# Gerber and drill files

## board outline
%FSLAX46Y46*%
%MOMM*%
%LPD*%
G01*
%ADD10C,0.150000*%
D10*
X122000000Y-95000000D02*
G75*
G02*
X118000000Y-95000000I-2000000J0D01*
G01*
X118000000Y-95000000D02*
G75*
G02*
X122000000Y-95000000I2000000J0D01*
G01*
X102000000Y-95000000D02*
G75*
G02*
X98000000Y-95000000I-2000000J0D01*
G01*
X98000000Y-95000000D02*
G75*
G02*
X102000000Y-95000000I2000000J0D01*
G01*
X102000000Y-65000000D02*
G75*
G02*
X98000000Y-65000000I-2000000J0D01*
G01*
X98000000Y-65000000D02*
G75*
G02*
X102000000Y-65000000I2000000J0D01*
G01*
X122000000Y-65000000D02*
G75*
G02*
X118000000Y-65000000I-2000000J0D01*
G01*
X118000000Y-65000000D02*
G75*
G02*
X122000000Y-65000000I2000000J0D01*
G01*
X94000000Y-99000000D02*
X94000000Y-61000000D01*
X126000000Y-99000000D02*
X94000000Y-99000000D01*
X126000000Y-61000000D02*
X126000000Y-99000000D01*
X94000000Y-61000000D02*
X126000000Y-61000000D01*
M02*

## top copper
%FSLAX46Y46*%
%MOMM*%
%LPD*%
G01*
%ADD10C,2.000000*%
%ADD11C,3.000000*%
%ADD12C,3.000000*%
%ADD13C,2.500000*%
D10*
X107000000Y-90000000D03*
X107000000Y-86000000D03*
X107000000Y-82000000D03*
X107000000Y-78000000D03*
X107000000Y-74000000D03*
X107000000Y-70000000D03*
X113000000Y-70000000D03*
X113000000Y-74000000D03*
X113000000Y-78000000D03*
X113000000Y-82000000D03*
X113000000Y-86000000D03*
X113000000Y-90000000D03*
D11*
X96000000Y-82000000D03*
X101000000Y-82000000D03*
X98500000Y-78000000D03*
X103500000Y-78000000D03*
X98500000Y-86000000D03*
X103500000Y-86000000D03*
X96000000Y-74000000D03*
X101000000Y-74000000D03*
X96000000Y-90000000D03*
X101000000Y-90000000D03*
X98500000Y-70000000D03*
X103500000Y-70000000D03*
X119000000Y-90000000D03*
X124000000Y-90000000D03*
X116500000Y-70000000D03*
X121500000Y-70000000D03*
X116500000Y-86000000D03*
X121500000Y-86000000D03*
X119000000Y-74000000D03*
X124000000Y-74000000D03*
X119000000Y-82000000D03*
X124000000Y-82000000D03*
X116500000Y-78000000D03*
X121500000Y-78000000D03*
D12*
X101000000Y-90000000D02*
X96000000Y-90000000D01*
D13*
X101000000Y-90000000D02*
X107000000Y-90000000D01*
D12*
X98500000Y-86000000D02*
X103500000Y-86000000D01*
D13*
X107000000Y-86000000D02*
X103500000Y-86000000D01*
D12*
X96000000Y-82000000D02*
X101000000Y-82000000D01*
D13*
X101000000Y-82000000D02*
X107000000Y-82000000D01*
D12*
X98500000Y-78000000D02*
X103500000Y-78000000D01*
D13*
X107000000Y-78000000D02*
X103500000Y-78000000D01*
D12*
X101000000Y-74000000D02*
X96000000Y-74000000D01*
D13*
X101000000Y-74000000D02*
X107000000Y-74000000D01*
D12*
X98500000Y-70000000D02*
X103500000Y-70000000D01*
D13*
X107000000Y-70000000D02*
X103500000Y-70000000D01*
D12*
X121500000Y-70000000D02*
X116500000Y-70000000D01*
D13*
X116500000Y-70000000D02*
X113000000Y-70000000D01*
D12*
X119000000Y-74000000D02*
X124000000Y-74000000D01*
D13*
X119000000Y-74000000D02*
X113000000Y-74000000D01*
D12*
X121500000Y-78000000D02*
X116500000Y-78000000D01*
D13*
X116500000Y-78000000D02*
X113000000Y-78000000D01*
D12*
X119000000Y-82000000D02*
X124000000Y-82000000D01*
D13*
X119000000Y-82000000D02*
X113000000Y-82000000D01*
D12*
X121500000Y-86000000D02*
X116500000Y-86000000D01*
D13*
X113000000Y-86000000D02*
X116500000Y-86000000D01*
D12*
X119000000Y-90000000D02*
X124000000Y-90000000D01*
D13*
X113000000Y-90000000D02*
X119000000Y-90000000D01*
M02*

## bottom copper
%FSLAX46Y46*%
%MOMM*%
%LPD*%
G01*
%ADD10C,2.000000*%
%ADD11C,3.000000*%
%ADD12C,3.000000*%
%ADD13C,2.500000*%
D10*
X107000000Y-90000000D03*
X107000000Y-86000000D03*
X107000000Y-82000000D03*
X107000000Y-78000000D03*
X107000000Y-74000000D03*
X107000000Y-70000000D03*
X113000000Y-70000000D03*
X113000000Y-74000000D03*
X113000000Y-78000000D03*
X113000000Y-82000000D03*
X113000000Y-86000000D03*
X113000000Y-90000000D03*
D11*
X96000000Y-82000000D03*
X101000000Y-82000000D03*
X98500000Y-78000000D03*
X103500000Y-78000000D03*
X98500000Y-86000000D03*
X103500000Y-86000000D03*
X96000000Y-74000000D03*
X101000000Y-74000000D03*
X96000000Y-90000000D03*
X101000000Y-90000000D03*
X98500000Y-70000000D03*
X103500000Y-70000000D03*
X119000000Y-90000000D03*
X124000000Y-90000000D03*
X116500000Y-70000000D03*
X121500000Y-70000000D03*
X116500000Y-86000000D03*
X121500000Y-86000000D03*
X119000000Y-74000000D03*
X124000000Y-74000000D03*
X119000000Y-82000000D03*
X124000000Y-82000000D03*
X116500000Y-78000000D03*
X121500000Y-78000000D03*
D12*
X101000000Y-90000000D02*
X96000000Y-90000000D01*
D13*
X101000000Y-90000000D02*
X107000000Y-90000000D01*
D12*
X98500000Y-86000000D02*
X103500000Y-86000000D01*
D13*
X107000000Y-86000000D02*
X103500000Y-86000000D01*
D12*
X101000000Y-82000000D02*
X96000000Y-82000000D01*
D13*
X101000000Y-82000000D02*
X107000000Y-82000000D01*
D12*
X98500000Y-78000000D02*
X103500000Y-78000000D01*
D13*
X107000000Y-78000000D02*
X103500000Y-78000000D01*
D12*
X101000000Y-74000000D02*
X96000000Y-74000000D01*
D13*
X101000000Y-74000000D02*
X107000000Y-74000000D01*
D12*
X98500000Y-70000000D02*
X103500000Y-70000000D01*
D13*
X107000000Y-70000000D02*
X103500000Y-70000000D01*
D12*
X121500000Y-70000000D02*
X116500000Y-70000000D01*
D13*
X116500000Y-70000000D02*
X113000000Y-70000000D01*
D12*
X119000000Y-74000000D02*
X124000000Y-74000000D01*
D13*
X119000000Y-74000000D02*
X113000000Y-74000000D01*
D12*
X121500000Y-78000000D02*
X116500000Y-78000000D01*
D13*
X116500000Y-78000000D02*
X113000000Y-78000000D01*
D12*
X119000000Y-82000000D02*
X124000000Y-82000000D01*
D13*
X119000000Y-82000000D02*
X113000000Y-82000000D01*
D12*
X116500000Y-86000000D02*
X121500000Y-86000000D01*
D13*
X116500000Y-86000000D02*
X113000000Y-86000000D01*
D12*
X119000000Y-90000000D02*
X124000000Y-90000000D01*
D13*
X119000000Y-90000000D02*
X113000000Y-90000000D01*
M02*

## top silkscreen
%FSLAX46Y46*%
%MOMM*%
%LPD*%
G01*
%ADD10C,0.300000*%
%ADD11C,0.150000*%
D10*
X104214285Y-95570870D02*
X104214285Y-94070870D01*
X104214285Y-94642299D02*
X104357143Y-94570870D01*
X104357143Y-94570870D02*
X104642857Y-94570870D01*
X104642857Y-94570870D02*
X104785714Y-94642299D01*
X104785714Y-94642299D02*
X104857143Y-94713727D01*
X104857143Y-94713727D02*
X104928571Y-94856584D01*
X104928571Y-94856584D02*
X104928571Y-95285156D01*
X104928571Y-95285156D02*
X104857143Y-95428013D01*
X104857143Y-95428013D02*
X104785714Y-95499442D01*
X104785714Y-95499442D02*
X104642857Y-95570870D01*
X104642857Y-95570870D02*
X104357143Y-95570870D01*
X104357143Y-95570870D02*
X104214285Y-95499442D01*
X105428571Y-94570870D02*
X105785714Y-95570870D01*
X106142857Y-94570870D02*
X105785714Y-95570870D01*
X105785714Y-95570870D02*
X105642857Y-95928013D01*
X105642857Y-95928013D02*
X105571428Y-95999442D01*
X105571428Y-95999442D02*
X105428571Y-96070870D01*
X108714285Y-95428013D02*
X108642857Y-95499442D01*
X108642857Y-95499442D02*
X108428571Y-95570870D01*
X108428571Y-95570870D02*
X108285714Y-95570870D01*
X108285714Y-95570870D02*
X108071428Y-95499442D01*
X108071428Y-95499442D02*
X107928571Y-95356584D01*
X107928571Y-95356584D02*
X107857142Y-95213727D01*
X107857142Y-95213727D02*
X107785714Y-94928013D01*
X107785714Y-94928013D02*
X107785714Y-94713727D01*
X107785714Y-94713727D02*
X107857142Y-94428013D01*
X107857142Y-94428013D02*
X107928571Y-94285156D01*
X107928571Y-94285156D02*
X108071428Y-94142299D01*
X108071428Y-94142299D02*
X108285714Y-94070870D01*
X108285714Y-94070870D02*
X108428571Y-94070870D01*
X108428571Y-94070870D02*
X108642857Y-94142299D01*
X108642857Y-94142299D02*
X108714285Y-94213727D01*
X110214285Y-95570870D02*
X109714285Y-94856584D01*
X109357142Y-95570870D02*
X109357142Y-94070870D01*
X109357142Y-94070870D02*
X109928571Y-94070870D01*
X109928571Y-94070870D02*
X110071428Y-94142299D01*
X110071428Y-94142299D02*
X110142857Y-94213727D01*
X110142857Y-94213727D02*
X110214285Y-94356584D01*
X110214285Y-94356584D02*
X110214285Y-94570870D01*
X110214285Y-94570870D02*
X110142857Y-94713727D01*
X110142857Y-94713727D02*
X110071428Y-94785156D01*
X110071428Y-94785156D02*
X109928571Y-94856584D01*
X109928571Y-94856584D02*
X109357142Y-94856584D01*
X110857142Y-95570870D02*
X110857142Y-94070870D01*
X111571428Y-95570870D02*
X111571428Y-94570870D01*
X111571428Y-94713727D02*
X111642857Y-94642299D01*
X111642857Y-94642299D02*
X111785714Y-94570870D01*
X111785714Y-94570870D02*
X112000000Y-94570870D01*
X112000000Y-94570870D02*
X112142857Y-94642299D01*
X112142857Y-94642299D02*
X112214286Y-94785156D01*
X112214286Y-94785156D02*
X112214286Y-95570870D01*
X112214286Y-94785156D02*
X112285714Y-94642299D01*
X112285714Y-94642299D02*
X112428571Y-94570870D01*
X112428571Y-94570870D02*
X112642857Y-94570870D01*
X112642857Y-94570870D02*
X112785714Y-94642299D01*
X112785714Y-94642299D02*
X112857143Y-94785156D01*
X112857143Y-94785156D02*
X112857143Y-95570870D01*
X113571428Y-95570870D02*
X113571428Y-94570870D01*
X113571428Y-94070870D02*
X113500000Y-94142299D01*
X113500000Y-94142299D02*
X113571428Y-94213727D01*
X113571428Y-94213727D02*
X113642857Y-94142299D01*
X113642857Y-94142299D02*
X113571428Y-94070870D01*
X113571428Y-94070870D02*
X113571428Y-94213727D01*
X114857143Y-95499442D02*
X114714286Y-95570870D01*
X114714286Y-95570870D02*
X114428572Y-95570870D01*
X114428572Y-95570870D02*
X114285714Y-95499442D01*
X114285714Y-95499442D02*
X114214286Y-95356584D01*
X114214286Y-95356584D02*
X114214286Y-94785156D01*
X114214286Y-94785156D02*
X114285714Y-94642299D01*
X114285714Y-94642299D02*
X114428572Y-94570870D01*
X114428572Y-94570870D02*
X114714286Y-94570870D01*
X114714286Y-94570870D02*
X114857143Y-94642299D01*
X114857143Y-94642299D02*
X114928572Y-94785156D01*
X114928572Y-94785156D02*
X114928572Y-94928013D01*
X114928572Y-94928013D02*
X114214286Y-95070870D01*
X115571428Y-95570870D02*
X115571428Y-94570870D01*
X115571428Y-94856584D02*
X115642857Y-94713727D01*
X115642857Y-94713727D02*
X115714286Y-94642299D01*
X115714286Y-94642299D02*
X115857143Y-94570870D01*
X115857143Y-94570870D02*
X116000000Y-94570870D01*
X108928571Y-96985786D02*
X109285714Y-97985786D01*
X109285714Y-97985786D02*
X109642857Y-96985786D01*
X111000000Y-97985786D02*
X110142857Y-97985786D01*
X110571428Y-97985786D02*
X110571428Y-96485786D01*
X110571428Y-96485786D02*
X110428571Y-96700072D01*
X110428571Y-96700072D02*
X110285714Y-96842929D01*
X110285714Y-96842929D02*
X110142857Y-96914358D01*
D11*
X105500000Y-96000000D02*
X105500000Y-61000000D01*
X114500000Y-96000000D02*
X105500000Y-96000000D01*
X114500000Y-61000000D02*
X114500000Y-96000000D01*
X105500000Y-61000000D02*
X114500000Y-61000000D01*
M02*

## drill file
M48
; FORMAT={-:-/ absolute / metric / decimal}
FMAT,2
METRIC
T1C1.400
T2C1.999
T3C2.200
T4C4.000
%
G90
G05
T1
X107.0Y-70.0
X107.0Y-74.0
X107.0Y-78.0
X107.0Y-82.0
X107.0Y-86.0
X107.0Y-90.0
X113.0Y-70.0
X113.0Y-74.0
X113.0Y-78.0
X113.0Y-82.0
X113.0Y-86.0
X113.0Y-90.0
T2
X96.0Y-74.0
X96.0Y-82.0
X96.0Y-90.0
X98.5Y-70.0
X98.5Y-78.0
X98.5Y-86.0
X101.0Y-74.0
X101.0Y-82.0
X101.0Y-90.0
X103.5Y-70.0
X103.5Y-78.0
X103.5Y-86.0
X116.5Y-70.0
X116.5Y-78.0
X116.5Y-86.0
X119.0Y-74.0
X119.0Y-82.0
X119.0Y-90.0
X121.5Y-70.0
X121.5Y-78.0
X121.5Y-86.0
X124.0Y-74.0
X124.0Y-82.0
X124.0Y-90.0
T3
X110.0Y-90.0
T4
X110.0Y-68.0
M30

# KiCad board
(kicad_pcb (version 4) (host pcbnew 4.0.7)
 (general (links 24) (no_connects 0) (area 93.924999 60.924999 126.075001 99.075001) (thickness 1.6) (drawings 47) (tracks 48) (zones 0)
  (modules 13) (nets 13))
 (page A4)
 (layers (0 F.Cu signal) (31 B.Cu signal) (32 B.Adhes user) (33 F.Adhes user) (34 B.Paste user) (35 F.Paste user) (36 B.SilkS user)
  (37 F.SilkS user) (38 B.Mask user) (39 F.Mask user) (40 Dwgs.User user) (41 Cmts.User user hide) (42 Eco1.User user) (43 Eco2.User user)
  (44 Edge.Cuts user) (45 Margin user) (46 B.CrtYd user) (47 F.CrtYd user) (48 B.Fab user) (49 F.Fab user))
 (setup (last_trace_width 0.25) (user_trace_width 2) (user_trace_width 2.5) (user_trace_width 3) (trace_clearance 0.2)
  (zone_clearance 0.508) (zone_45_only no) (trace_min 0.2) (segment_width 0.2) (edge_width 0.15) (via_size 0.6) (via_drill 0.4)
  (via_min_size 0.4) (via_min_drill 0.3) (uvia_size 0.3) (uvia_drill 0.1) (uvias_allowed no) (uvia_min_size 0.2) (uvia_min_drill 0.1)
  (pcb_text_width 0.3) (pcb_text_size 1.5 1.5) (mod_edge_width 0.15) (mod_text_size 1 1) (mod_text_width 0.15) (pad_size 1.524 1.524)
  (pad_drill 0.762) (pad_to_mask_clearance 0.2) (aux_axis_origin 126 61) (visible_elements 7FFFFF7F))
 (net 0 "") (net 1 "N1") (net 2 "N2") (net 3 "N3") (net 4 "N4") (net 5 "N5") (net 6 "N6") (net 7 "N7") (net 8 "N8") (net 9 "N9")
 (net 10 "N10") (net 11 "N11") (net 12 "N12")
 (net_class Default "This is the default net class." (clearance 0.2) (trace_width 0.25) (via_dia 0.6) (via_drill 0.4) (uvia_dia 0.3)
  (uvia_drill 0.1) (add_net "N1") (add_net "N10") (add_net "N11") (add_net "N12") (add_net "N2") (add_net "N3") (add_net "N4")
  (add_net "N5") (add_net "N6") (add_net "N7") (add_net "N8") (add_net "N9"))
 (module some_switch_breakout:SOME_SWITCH (layer F.Cu) (at 110 80)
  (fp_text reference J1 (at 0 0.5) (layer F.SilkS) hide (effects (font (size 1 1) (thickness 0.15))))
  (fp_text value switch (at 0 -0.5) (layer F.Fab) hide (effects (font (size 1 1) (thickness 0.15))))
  (fp_line (start -4.5 16) (end -4.5 -19) (layer F.SilkS) (width 0.15))
  (fp_line (start 4.5 16) (end -4.5 16) (layer F.SilkS) (width 0.15))
  (fp_line (start 4.5 -19) (end 4.5 16) (layer F.SilkS) (width 0.15))
  (fp_line (start -4.5 -19) (end 4.5 -19) (layer F.SilkS) (width 0.15))
  (pad 1 thru_hole circle (at -3 10) (size 2 2) (drill 1.4) (layers *.Cu *.Mask) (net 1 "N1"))
  (pad 2 thru_hole circle (at -3 6) (size 2 2) (drill 1.4) (layers *.Cu *.Mask) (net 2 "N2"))
  (pad 3 thru_hole circle (at -3 2) (size 2 2) (drill 1.4) (layers *.Cu *.Mask) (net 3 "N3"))
  (pad 4 thru_hole circle (at -3 -2) (size 2 2) (drill 1.4) (layers *.Cu *.Mask) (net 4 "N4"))
  (pad 5 thru_hole circle (at -3 -6) (size 2 2) (drill 1.4) (layers *.Cu *.Mask) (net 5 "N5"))
  (pad 6 thru_hole circle (at -3 -10) (size 2 2) (drill 1.4) (layers *.Cu *.Mask) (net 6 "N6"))
  (pad 7 thru_hole circle (at 3 -10) (size 2 2) (drill 1.4) (layers *.Cu *.Mask) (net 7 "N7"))
  (pad 8 thru_hole circle (at 3 -6) (size 2 2) (drill 1.4) (layers *.Cu *.Mask) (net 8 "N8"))
  (pad 9 thru_hole circle (at 3 -2) (size 2 2) (drill 1.4) (layers *.Cu *.Mask) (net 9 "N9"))
  (pad 10 thru_hole circle (at 3 2) (size 2 2) (drill 1.4) (layers *.Cu *.Mask) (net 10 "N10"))
  (pad 11 thru_hole circle (at 3 6) (size 2 2) (drill 1.4) (layers *.Cu *.Mask) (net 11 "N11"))
  (pad 12 thru_hole circle (at 3 10) (size 2 2) (drill 1.4) (layers *.Cu *.Mask) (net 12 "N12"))
  (pad "" np_thru_hole circle (at 0 10) (size 2.2 2.2) (drill 2.2) (layers *.Cu *.Mask))
  (pad "" np_thru_hole circle (at 0 -12) (size 4 4) (drill 4) (layers *.Cu *.Mask)))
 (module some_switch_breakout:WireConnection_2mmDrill (layer F.Cu) (at 98.5 82)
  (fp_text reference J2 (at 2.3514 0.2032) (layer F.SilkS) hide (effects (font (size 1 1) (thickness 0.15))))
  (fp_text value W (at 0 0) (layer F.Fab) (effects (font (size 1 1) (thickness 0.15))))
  (pad 1 thru_hole circle (at -2.5 0) (size 3 3) (drill 1.99898) (layers *.Cu *.Mask) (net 3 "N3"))
  (pad 2 thru_hole circle (at 2.5 0) (size 3 3) (drill 1.99898) (layers *.Cu *.Mask) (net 3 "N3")))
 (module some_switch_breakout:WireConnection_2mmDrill (layer F.Cu) (at 101 78)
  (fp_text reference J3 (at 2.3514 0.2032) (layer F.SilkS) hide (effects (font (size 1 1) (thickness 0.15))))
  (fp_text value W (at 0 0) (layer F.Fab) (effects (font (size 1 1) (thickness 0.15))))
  (pad 1 thru_hole circle (at -2.5 0) (size 3 3) (drill 1.99898) (layers *.Cu *.Mask) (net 4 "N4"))
  (pad 2 thru_hole circle (at 2.5 0) (size 3 3) (drill 1.99898) (layers *.Cu *.Mask) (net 4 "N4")))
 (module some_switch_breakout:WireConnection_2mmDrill (layer F.Cu) (at 101 86)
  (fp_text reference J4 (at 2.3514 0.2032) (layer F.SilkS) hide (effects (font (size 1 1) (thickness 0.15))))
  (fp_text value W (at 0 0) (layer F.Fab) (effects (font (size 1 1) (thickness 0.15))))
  (pad 1 thru_hole circle (at -2.5 0) (size 3 3) (drill 1.99898) (layers *.Cu *.Mask) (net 2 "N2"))
  (pad 2 thru_hole circle (at 2.5 0) (size 3 3) (drill 1.99898) (layers *.Cu *.Mask) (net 2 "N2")))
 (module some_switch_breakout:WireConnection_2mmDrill (layer F.Cu) (at 98.5 74)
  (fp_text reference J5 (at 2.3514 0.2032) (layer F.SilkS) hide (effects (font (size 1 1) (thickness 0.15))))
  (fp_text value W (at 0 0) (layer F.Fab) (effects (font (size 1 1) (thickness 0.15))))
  (pad 1 thru_hole circle (at -2.5 0) (size 3 3) (drill 1.99898) (layers *.Cu *.Mask) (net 5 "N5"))
  (pad 2 thru_hole circle (at 2.5 0) (size 3 3) (drill 1.99898) (layers *.Cu *.Mask) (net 5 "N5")))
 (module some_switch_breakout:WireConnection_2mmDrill (layer F.Cu) (at 98.5 90)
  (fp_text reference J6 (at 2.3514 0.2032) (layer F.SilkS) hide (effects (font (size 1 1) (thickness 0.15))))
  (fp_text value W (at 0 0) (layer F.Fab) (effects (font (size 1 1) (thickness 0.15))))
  (pad 1 thru_hole circle (at -2.5 0) (size 3 3) (drill 1.99898) (layers *.Cu *.Mask) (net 1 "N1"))
  (pad 2 thru_hole circle (at 2.5 0) (size 3 3) (drill 1.99898) (layers *.Cu *.Mask) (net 1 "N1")))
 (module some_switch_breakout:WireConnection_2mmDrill (layer F.Cu) (at 101 70)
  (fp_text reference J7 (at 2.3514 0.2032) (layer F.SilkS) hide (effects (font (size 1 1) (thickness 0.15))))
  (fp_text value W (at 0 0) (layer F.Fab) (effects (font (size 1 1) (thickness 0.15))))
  (pad 1 thru_hole circle (at -2.5 0) (size 3 3) (drill 1.99898) (layers *.Cu *.Mask) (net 6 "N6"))
  (pad 2 thru_hole circle (at 2.5 0) (size 3 3) (drill 1.99898) (layers *.Cu *.Mask) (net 6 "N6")))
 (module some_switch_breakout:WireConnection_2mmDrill (layer F.Cu) (at 121.5 90)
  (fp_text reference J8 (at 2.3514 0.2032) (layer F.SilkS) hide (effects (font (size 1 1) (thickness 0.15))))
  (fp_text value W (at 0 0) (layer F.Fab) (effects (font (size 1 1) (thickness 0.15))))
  (pad 1 thru_hole circle (at -2.5 0) (size 3 3) (drill 1.99898) (layers *.Cu *.Mask) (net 12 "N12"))
  (pad 2 thru_hole circle (at 2.5 0) (size 3 3) (drill 1.99898) (layers *.Cu *.Mask) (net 12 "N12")))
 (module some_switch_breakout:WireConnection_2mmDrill (layer F.Cu) (at 119 70)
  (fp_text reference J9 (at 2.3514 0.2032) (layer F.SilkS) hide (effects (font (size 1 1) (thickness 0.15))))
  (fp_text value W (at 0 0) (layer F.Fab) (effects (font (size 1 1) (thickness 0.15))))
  (pad 1 thru_hole circle (at -2.5 0) (size 3 3) (drill 1.99898) (layers *.Cu *.Mask) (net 7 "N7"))
  (pad 2 thru_hole circle (at 2.5 0) (size 3 3) (drill 1.99898) (layers *.Cu *.Mask) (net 7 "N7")))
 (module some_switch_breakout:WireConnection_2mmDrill (layer F.Cu) (at 119 86)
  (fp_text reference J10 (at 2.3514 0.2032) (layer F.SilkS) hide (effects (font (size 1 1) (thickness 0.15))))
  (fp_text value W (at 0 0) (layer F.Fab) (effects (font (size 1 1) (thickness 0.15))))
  (pad 1 thru_hole circle (at -2.5 0) (size 3 3) (drill 1.99898) (layers *.Cu *.Mask) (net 11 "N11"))
  (pad 2 thru_hole circle (at 2.5 0) (size 3 3) (drill 1.99898) (layers *.Cu *.Mask) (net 11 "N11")))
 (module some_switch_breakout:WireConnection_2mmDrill (layer F.Cu) (at 121.5 74)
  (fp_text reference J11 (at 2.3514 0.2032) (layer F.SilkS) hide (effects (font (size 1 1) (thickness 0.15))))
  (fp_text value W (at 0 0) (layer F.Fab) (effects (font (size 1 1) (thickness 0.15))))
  (pad 1 thru_hole circle (at -2.5 0) (size 3 3) (drill 1.99898) (layers *.Cu *.Mask) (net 8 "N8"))
  (pad 2 thru_hole circle (at 2.5 0) (size 3 3) (drill 1.99898) (layers *.Cu *.Mask) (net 8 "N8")))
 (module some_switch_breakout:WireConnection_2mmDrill (layer F.Cu) (at 121.5 82)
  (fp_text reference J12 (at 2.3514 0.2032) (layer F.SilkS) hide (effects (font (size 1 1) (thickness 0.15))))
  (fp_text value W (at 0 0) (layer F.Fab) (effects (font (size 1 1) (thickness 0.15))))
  (pad 1 thru_hole circle (at -2.5 0) (size 3 3) (drill 1.99898) (layers *.Cu *.Mask) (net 10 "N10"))
  (pad 2 thru_hole circle (at 2.5 0) (size 3 3) (drill 1.99898) (layers *.Cu *.Mask) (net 10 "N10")))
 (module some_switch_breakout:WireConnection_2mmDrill (layer F.Cu) (at 119 78)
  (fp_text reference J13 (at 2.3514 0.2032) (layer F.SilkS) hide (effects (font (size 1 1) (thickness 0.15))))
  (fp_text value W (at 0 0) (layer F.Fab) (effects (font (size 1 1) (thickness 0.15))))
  (pad 1 thru_hole circle (at -2.5 0) (size 3 3) (drill 1.99898) (layers *.Cu *.Mask) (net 9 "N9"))
  (pad 2 thru_hole circle (at 2.5 0) (size 3 3) (drill 1.99898) (layers *.Cu *.Mask) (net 9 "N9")))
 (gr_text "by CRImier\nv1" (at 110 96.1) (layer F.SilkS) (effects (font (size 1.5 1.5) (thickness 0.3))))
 (gr_circle (center 120 95) (end 122 95) (layer Edge.Cuts) (width 0.15))
 (gr_circle (center 100 95) (end 102 95) (layer Edge.Cuts) (width 0.15))
 (gr_circle (center 100 65) (end 102 65) (layer Edge.Cuts) (width 0.15))
 (gr_circle (center 120 65) (end 122 65) (layer Edge.Cuts) (width 0.15))
 (gr_line (start 94 99) (end 94 61) (layer Edge.Cuts) (width 0.15))
 (gr_line (start 126 99) (end 94 99) (layer Edge.Cuts) (width 0.15))
 (gr_line (start 126 61) (end 126 99) (layer Edge.Cuts) (width 0.15))
 (gr_line (start 94 61) (end 126 61) (layer Edge.Cuts) (width 0.15))
 (segment (start 101 90) (end 96 90) (width 3) (layer F.Cu) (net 1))
 (segment (start 101 90) (end 96 90) (width 3) (layer B.Cu) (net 1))
 (segment (start 101 90) (end 107 90) (width 2.5) (layer B.Cu) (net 1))
 (segment (start 101 90) (end 107 90) (width 2.5) (layer F.Cu) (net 1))
 (segment (start 98.5 86) (end 103.5 86) (width 3) (layer F.Cu) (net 2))
 (segment (start 98.5 86) (end 103.5 86) (width 3) (layer B.Cu) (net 2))
 (segment (start 107 86) (end 103.5 86) (width 2.5) (layer B.Cu) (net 2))
 (segment (start 107 86) (end 103.5 86) (width 2.5) (layer F.Cu) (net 2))
 (segment (start 96 82) (end 101 82) (width 3) (layer F.Cu) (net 3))
 (segment (start 101 82) (end 96 82) (width 3) (layer B.Cu) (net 3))
 (segment (start 101 82) (end 107 82) (width 2.5) (layer B.Cu) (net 3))
 (segment (start 101 82) (end 107 82) (width 2.5) (layer F.Cu) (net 3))
 (segment (start 98.5 78) (end 103.5 78) (width 3) (layer F.Cu) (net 4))
 (segment (start 98.5 78) (end 103.5 78) (width 3) (layer B.Cu) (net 4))
 (segment (start 107 78) (end 103.5 78) (width 2.5) (layer B.Cu) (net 4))
 (segment (start 107 78) (end 103.5 78) (width 2.5) (layer F.Cu) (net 4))
 (segment (start 101 74) (end 96 74) (width 3) (layer F.Cu) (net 5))
 (segment (start 101 74) (end 96 74) (width 3) (layer B.Cu) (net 5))
 (segment (start 101 74) (end 107 74) (width 2.5) (layer B.Cu) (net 5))
 (segment (start 101 74) (end 107 74) (width 2.5) (layer F.Cu) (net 5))
 (segment (start 98.5 70) (end 103.5 70) (width 3) (layer F.Cu) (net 6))
 (segment (start 98.5 70) (end 103.5 70) (width 3) (layer B.Cu) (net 6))
 (segment (start 107 70) (end 103.5 70) (width 2.5) (layer B.Cu) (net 6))
 (segment (start 107 70) (end 103.5 70) (width 2.5) (layer F.Cu) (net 6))
 (segment (start 121.5 70) (end 116.5 70) (width 3) (layer F.Cu) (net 7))
 (segment (start 121.5 70) (end 116.5 70) (width 3) (layer B.Cu) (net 7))
 (segment (start 116.5 70) (end 113 70) (width 2.5) (layer B.Cu) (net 7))
 (segment (start 116.5 70) (end 113 70) (width 2.5) (layer F.Cu) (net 7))
 (segment (start 119 74) (end 124 74) (width 3) (layer F.Cu) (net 8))
 (segment (start 119 74) (end 124 74) (width 3) (layer B.Cu) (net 8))
 (segment (start 119 74) (end 113 74) (width 2.5) (layer B.Cu) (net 8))
 (segment (start 119 74) (end 113 74) (width 2.5) (layer F.Cu) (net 8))
 (segment (start 121.5 78) (end 116.5 78) (width 3) (layer F.Cu) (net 9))
 (segment (start 121.5 78) (end 116.5 78) (width 3) (layer B.Cu) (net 9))
 (segment (start 116.5 78) (end 113 78) (width 2.5) (layer B.Cu) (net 9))
 (segment (start 116.5 78) (end 113 78) (width 2.5) (layer F.Cu) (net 9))
 (segment (start 119 82) (end 124 82) (width 3) (layer F.Cu) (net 10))
 (segment (start 119 82) (end 124 82) (width 3) (layer B.Cu) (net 10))
 (segment (start 119 82) (end 113 82) (width 2.5) (layer B.Cu) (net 10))
 (segment (start 119 82) (end 113 82) (width 2.5) (layer F.Cu) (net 10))
 (segment (start 121.5 86) (end 116.5 86) (width 3) (layer F.Cu) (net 11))
 (segment (start 116.5 86) (end 121.5 86) (width 3) (layer B.Cu) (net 11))
 (segment (start 116.5 86) (end 113 86) (width 2.5) (layer B.Cu) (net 11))
 (segment (start 113 86) (end 116.5 86) (width 2.5) (layer F.Cu) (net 11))
 (segment (start 119 90) (end 124 90) (width 3) (layer F.Cu) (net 12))
 (segment (start 119 90) (end 124 90) (width 3) (layer B.Cu) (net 12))
 (segment (start 119 90) (end 113 90) (width 2.5) (layer B.Cu) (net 12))
 (segment (start 113 90) (end 119 90) (width 2.5) (layer F.Cu) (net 12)))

